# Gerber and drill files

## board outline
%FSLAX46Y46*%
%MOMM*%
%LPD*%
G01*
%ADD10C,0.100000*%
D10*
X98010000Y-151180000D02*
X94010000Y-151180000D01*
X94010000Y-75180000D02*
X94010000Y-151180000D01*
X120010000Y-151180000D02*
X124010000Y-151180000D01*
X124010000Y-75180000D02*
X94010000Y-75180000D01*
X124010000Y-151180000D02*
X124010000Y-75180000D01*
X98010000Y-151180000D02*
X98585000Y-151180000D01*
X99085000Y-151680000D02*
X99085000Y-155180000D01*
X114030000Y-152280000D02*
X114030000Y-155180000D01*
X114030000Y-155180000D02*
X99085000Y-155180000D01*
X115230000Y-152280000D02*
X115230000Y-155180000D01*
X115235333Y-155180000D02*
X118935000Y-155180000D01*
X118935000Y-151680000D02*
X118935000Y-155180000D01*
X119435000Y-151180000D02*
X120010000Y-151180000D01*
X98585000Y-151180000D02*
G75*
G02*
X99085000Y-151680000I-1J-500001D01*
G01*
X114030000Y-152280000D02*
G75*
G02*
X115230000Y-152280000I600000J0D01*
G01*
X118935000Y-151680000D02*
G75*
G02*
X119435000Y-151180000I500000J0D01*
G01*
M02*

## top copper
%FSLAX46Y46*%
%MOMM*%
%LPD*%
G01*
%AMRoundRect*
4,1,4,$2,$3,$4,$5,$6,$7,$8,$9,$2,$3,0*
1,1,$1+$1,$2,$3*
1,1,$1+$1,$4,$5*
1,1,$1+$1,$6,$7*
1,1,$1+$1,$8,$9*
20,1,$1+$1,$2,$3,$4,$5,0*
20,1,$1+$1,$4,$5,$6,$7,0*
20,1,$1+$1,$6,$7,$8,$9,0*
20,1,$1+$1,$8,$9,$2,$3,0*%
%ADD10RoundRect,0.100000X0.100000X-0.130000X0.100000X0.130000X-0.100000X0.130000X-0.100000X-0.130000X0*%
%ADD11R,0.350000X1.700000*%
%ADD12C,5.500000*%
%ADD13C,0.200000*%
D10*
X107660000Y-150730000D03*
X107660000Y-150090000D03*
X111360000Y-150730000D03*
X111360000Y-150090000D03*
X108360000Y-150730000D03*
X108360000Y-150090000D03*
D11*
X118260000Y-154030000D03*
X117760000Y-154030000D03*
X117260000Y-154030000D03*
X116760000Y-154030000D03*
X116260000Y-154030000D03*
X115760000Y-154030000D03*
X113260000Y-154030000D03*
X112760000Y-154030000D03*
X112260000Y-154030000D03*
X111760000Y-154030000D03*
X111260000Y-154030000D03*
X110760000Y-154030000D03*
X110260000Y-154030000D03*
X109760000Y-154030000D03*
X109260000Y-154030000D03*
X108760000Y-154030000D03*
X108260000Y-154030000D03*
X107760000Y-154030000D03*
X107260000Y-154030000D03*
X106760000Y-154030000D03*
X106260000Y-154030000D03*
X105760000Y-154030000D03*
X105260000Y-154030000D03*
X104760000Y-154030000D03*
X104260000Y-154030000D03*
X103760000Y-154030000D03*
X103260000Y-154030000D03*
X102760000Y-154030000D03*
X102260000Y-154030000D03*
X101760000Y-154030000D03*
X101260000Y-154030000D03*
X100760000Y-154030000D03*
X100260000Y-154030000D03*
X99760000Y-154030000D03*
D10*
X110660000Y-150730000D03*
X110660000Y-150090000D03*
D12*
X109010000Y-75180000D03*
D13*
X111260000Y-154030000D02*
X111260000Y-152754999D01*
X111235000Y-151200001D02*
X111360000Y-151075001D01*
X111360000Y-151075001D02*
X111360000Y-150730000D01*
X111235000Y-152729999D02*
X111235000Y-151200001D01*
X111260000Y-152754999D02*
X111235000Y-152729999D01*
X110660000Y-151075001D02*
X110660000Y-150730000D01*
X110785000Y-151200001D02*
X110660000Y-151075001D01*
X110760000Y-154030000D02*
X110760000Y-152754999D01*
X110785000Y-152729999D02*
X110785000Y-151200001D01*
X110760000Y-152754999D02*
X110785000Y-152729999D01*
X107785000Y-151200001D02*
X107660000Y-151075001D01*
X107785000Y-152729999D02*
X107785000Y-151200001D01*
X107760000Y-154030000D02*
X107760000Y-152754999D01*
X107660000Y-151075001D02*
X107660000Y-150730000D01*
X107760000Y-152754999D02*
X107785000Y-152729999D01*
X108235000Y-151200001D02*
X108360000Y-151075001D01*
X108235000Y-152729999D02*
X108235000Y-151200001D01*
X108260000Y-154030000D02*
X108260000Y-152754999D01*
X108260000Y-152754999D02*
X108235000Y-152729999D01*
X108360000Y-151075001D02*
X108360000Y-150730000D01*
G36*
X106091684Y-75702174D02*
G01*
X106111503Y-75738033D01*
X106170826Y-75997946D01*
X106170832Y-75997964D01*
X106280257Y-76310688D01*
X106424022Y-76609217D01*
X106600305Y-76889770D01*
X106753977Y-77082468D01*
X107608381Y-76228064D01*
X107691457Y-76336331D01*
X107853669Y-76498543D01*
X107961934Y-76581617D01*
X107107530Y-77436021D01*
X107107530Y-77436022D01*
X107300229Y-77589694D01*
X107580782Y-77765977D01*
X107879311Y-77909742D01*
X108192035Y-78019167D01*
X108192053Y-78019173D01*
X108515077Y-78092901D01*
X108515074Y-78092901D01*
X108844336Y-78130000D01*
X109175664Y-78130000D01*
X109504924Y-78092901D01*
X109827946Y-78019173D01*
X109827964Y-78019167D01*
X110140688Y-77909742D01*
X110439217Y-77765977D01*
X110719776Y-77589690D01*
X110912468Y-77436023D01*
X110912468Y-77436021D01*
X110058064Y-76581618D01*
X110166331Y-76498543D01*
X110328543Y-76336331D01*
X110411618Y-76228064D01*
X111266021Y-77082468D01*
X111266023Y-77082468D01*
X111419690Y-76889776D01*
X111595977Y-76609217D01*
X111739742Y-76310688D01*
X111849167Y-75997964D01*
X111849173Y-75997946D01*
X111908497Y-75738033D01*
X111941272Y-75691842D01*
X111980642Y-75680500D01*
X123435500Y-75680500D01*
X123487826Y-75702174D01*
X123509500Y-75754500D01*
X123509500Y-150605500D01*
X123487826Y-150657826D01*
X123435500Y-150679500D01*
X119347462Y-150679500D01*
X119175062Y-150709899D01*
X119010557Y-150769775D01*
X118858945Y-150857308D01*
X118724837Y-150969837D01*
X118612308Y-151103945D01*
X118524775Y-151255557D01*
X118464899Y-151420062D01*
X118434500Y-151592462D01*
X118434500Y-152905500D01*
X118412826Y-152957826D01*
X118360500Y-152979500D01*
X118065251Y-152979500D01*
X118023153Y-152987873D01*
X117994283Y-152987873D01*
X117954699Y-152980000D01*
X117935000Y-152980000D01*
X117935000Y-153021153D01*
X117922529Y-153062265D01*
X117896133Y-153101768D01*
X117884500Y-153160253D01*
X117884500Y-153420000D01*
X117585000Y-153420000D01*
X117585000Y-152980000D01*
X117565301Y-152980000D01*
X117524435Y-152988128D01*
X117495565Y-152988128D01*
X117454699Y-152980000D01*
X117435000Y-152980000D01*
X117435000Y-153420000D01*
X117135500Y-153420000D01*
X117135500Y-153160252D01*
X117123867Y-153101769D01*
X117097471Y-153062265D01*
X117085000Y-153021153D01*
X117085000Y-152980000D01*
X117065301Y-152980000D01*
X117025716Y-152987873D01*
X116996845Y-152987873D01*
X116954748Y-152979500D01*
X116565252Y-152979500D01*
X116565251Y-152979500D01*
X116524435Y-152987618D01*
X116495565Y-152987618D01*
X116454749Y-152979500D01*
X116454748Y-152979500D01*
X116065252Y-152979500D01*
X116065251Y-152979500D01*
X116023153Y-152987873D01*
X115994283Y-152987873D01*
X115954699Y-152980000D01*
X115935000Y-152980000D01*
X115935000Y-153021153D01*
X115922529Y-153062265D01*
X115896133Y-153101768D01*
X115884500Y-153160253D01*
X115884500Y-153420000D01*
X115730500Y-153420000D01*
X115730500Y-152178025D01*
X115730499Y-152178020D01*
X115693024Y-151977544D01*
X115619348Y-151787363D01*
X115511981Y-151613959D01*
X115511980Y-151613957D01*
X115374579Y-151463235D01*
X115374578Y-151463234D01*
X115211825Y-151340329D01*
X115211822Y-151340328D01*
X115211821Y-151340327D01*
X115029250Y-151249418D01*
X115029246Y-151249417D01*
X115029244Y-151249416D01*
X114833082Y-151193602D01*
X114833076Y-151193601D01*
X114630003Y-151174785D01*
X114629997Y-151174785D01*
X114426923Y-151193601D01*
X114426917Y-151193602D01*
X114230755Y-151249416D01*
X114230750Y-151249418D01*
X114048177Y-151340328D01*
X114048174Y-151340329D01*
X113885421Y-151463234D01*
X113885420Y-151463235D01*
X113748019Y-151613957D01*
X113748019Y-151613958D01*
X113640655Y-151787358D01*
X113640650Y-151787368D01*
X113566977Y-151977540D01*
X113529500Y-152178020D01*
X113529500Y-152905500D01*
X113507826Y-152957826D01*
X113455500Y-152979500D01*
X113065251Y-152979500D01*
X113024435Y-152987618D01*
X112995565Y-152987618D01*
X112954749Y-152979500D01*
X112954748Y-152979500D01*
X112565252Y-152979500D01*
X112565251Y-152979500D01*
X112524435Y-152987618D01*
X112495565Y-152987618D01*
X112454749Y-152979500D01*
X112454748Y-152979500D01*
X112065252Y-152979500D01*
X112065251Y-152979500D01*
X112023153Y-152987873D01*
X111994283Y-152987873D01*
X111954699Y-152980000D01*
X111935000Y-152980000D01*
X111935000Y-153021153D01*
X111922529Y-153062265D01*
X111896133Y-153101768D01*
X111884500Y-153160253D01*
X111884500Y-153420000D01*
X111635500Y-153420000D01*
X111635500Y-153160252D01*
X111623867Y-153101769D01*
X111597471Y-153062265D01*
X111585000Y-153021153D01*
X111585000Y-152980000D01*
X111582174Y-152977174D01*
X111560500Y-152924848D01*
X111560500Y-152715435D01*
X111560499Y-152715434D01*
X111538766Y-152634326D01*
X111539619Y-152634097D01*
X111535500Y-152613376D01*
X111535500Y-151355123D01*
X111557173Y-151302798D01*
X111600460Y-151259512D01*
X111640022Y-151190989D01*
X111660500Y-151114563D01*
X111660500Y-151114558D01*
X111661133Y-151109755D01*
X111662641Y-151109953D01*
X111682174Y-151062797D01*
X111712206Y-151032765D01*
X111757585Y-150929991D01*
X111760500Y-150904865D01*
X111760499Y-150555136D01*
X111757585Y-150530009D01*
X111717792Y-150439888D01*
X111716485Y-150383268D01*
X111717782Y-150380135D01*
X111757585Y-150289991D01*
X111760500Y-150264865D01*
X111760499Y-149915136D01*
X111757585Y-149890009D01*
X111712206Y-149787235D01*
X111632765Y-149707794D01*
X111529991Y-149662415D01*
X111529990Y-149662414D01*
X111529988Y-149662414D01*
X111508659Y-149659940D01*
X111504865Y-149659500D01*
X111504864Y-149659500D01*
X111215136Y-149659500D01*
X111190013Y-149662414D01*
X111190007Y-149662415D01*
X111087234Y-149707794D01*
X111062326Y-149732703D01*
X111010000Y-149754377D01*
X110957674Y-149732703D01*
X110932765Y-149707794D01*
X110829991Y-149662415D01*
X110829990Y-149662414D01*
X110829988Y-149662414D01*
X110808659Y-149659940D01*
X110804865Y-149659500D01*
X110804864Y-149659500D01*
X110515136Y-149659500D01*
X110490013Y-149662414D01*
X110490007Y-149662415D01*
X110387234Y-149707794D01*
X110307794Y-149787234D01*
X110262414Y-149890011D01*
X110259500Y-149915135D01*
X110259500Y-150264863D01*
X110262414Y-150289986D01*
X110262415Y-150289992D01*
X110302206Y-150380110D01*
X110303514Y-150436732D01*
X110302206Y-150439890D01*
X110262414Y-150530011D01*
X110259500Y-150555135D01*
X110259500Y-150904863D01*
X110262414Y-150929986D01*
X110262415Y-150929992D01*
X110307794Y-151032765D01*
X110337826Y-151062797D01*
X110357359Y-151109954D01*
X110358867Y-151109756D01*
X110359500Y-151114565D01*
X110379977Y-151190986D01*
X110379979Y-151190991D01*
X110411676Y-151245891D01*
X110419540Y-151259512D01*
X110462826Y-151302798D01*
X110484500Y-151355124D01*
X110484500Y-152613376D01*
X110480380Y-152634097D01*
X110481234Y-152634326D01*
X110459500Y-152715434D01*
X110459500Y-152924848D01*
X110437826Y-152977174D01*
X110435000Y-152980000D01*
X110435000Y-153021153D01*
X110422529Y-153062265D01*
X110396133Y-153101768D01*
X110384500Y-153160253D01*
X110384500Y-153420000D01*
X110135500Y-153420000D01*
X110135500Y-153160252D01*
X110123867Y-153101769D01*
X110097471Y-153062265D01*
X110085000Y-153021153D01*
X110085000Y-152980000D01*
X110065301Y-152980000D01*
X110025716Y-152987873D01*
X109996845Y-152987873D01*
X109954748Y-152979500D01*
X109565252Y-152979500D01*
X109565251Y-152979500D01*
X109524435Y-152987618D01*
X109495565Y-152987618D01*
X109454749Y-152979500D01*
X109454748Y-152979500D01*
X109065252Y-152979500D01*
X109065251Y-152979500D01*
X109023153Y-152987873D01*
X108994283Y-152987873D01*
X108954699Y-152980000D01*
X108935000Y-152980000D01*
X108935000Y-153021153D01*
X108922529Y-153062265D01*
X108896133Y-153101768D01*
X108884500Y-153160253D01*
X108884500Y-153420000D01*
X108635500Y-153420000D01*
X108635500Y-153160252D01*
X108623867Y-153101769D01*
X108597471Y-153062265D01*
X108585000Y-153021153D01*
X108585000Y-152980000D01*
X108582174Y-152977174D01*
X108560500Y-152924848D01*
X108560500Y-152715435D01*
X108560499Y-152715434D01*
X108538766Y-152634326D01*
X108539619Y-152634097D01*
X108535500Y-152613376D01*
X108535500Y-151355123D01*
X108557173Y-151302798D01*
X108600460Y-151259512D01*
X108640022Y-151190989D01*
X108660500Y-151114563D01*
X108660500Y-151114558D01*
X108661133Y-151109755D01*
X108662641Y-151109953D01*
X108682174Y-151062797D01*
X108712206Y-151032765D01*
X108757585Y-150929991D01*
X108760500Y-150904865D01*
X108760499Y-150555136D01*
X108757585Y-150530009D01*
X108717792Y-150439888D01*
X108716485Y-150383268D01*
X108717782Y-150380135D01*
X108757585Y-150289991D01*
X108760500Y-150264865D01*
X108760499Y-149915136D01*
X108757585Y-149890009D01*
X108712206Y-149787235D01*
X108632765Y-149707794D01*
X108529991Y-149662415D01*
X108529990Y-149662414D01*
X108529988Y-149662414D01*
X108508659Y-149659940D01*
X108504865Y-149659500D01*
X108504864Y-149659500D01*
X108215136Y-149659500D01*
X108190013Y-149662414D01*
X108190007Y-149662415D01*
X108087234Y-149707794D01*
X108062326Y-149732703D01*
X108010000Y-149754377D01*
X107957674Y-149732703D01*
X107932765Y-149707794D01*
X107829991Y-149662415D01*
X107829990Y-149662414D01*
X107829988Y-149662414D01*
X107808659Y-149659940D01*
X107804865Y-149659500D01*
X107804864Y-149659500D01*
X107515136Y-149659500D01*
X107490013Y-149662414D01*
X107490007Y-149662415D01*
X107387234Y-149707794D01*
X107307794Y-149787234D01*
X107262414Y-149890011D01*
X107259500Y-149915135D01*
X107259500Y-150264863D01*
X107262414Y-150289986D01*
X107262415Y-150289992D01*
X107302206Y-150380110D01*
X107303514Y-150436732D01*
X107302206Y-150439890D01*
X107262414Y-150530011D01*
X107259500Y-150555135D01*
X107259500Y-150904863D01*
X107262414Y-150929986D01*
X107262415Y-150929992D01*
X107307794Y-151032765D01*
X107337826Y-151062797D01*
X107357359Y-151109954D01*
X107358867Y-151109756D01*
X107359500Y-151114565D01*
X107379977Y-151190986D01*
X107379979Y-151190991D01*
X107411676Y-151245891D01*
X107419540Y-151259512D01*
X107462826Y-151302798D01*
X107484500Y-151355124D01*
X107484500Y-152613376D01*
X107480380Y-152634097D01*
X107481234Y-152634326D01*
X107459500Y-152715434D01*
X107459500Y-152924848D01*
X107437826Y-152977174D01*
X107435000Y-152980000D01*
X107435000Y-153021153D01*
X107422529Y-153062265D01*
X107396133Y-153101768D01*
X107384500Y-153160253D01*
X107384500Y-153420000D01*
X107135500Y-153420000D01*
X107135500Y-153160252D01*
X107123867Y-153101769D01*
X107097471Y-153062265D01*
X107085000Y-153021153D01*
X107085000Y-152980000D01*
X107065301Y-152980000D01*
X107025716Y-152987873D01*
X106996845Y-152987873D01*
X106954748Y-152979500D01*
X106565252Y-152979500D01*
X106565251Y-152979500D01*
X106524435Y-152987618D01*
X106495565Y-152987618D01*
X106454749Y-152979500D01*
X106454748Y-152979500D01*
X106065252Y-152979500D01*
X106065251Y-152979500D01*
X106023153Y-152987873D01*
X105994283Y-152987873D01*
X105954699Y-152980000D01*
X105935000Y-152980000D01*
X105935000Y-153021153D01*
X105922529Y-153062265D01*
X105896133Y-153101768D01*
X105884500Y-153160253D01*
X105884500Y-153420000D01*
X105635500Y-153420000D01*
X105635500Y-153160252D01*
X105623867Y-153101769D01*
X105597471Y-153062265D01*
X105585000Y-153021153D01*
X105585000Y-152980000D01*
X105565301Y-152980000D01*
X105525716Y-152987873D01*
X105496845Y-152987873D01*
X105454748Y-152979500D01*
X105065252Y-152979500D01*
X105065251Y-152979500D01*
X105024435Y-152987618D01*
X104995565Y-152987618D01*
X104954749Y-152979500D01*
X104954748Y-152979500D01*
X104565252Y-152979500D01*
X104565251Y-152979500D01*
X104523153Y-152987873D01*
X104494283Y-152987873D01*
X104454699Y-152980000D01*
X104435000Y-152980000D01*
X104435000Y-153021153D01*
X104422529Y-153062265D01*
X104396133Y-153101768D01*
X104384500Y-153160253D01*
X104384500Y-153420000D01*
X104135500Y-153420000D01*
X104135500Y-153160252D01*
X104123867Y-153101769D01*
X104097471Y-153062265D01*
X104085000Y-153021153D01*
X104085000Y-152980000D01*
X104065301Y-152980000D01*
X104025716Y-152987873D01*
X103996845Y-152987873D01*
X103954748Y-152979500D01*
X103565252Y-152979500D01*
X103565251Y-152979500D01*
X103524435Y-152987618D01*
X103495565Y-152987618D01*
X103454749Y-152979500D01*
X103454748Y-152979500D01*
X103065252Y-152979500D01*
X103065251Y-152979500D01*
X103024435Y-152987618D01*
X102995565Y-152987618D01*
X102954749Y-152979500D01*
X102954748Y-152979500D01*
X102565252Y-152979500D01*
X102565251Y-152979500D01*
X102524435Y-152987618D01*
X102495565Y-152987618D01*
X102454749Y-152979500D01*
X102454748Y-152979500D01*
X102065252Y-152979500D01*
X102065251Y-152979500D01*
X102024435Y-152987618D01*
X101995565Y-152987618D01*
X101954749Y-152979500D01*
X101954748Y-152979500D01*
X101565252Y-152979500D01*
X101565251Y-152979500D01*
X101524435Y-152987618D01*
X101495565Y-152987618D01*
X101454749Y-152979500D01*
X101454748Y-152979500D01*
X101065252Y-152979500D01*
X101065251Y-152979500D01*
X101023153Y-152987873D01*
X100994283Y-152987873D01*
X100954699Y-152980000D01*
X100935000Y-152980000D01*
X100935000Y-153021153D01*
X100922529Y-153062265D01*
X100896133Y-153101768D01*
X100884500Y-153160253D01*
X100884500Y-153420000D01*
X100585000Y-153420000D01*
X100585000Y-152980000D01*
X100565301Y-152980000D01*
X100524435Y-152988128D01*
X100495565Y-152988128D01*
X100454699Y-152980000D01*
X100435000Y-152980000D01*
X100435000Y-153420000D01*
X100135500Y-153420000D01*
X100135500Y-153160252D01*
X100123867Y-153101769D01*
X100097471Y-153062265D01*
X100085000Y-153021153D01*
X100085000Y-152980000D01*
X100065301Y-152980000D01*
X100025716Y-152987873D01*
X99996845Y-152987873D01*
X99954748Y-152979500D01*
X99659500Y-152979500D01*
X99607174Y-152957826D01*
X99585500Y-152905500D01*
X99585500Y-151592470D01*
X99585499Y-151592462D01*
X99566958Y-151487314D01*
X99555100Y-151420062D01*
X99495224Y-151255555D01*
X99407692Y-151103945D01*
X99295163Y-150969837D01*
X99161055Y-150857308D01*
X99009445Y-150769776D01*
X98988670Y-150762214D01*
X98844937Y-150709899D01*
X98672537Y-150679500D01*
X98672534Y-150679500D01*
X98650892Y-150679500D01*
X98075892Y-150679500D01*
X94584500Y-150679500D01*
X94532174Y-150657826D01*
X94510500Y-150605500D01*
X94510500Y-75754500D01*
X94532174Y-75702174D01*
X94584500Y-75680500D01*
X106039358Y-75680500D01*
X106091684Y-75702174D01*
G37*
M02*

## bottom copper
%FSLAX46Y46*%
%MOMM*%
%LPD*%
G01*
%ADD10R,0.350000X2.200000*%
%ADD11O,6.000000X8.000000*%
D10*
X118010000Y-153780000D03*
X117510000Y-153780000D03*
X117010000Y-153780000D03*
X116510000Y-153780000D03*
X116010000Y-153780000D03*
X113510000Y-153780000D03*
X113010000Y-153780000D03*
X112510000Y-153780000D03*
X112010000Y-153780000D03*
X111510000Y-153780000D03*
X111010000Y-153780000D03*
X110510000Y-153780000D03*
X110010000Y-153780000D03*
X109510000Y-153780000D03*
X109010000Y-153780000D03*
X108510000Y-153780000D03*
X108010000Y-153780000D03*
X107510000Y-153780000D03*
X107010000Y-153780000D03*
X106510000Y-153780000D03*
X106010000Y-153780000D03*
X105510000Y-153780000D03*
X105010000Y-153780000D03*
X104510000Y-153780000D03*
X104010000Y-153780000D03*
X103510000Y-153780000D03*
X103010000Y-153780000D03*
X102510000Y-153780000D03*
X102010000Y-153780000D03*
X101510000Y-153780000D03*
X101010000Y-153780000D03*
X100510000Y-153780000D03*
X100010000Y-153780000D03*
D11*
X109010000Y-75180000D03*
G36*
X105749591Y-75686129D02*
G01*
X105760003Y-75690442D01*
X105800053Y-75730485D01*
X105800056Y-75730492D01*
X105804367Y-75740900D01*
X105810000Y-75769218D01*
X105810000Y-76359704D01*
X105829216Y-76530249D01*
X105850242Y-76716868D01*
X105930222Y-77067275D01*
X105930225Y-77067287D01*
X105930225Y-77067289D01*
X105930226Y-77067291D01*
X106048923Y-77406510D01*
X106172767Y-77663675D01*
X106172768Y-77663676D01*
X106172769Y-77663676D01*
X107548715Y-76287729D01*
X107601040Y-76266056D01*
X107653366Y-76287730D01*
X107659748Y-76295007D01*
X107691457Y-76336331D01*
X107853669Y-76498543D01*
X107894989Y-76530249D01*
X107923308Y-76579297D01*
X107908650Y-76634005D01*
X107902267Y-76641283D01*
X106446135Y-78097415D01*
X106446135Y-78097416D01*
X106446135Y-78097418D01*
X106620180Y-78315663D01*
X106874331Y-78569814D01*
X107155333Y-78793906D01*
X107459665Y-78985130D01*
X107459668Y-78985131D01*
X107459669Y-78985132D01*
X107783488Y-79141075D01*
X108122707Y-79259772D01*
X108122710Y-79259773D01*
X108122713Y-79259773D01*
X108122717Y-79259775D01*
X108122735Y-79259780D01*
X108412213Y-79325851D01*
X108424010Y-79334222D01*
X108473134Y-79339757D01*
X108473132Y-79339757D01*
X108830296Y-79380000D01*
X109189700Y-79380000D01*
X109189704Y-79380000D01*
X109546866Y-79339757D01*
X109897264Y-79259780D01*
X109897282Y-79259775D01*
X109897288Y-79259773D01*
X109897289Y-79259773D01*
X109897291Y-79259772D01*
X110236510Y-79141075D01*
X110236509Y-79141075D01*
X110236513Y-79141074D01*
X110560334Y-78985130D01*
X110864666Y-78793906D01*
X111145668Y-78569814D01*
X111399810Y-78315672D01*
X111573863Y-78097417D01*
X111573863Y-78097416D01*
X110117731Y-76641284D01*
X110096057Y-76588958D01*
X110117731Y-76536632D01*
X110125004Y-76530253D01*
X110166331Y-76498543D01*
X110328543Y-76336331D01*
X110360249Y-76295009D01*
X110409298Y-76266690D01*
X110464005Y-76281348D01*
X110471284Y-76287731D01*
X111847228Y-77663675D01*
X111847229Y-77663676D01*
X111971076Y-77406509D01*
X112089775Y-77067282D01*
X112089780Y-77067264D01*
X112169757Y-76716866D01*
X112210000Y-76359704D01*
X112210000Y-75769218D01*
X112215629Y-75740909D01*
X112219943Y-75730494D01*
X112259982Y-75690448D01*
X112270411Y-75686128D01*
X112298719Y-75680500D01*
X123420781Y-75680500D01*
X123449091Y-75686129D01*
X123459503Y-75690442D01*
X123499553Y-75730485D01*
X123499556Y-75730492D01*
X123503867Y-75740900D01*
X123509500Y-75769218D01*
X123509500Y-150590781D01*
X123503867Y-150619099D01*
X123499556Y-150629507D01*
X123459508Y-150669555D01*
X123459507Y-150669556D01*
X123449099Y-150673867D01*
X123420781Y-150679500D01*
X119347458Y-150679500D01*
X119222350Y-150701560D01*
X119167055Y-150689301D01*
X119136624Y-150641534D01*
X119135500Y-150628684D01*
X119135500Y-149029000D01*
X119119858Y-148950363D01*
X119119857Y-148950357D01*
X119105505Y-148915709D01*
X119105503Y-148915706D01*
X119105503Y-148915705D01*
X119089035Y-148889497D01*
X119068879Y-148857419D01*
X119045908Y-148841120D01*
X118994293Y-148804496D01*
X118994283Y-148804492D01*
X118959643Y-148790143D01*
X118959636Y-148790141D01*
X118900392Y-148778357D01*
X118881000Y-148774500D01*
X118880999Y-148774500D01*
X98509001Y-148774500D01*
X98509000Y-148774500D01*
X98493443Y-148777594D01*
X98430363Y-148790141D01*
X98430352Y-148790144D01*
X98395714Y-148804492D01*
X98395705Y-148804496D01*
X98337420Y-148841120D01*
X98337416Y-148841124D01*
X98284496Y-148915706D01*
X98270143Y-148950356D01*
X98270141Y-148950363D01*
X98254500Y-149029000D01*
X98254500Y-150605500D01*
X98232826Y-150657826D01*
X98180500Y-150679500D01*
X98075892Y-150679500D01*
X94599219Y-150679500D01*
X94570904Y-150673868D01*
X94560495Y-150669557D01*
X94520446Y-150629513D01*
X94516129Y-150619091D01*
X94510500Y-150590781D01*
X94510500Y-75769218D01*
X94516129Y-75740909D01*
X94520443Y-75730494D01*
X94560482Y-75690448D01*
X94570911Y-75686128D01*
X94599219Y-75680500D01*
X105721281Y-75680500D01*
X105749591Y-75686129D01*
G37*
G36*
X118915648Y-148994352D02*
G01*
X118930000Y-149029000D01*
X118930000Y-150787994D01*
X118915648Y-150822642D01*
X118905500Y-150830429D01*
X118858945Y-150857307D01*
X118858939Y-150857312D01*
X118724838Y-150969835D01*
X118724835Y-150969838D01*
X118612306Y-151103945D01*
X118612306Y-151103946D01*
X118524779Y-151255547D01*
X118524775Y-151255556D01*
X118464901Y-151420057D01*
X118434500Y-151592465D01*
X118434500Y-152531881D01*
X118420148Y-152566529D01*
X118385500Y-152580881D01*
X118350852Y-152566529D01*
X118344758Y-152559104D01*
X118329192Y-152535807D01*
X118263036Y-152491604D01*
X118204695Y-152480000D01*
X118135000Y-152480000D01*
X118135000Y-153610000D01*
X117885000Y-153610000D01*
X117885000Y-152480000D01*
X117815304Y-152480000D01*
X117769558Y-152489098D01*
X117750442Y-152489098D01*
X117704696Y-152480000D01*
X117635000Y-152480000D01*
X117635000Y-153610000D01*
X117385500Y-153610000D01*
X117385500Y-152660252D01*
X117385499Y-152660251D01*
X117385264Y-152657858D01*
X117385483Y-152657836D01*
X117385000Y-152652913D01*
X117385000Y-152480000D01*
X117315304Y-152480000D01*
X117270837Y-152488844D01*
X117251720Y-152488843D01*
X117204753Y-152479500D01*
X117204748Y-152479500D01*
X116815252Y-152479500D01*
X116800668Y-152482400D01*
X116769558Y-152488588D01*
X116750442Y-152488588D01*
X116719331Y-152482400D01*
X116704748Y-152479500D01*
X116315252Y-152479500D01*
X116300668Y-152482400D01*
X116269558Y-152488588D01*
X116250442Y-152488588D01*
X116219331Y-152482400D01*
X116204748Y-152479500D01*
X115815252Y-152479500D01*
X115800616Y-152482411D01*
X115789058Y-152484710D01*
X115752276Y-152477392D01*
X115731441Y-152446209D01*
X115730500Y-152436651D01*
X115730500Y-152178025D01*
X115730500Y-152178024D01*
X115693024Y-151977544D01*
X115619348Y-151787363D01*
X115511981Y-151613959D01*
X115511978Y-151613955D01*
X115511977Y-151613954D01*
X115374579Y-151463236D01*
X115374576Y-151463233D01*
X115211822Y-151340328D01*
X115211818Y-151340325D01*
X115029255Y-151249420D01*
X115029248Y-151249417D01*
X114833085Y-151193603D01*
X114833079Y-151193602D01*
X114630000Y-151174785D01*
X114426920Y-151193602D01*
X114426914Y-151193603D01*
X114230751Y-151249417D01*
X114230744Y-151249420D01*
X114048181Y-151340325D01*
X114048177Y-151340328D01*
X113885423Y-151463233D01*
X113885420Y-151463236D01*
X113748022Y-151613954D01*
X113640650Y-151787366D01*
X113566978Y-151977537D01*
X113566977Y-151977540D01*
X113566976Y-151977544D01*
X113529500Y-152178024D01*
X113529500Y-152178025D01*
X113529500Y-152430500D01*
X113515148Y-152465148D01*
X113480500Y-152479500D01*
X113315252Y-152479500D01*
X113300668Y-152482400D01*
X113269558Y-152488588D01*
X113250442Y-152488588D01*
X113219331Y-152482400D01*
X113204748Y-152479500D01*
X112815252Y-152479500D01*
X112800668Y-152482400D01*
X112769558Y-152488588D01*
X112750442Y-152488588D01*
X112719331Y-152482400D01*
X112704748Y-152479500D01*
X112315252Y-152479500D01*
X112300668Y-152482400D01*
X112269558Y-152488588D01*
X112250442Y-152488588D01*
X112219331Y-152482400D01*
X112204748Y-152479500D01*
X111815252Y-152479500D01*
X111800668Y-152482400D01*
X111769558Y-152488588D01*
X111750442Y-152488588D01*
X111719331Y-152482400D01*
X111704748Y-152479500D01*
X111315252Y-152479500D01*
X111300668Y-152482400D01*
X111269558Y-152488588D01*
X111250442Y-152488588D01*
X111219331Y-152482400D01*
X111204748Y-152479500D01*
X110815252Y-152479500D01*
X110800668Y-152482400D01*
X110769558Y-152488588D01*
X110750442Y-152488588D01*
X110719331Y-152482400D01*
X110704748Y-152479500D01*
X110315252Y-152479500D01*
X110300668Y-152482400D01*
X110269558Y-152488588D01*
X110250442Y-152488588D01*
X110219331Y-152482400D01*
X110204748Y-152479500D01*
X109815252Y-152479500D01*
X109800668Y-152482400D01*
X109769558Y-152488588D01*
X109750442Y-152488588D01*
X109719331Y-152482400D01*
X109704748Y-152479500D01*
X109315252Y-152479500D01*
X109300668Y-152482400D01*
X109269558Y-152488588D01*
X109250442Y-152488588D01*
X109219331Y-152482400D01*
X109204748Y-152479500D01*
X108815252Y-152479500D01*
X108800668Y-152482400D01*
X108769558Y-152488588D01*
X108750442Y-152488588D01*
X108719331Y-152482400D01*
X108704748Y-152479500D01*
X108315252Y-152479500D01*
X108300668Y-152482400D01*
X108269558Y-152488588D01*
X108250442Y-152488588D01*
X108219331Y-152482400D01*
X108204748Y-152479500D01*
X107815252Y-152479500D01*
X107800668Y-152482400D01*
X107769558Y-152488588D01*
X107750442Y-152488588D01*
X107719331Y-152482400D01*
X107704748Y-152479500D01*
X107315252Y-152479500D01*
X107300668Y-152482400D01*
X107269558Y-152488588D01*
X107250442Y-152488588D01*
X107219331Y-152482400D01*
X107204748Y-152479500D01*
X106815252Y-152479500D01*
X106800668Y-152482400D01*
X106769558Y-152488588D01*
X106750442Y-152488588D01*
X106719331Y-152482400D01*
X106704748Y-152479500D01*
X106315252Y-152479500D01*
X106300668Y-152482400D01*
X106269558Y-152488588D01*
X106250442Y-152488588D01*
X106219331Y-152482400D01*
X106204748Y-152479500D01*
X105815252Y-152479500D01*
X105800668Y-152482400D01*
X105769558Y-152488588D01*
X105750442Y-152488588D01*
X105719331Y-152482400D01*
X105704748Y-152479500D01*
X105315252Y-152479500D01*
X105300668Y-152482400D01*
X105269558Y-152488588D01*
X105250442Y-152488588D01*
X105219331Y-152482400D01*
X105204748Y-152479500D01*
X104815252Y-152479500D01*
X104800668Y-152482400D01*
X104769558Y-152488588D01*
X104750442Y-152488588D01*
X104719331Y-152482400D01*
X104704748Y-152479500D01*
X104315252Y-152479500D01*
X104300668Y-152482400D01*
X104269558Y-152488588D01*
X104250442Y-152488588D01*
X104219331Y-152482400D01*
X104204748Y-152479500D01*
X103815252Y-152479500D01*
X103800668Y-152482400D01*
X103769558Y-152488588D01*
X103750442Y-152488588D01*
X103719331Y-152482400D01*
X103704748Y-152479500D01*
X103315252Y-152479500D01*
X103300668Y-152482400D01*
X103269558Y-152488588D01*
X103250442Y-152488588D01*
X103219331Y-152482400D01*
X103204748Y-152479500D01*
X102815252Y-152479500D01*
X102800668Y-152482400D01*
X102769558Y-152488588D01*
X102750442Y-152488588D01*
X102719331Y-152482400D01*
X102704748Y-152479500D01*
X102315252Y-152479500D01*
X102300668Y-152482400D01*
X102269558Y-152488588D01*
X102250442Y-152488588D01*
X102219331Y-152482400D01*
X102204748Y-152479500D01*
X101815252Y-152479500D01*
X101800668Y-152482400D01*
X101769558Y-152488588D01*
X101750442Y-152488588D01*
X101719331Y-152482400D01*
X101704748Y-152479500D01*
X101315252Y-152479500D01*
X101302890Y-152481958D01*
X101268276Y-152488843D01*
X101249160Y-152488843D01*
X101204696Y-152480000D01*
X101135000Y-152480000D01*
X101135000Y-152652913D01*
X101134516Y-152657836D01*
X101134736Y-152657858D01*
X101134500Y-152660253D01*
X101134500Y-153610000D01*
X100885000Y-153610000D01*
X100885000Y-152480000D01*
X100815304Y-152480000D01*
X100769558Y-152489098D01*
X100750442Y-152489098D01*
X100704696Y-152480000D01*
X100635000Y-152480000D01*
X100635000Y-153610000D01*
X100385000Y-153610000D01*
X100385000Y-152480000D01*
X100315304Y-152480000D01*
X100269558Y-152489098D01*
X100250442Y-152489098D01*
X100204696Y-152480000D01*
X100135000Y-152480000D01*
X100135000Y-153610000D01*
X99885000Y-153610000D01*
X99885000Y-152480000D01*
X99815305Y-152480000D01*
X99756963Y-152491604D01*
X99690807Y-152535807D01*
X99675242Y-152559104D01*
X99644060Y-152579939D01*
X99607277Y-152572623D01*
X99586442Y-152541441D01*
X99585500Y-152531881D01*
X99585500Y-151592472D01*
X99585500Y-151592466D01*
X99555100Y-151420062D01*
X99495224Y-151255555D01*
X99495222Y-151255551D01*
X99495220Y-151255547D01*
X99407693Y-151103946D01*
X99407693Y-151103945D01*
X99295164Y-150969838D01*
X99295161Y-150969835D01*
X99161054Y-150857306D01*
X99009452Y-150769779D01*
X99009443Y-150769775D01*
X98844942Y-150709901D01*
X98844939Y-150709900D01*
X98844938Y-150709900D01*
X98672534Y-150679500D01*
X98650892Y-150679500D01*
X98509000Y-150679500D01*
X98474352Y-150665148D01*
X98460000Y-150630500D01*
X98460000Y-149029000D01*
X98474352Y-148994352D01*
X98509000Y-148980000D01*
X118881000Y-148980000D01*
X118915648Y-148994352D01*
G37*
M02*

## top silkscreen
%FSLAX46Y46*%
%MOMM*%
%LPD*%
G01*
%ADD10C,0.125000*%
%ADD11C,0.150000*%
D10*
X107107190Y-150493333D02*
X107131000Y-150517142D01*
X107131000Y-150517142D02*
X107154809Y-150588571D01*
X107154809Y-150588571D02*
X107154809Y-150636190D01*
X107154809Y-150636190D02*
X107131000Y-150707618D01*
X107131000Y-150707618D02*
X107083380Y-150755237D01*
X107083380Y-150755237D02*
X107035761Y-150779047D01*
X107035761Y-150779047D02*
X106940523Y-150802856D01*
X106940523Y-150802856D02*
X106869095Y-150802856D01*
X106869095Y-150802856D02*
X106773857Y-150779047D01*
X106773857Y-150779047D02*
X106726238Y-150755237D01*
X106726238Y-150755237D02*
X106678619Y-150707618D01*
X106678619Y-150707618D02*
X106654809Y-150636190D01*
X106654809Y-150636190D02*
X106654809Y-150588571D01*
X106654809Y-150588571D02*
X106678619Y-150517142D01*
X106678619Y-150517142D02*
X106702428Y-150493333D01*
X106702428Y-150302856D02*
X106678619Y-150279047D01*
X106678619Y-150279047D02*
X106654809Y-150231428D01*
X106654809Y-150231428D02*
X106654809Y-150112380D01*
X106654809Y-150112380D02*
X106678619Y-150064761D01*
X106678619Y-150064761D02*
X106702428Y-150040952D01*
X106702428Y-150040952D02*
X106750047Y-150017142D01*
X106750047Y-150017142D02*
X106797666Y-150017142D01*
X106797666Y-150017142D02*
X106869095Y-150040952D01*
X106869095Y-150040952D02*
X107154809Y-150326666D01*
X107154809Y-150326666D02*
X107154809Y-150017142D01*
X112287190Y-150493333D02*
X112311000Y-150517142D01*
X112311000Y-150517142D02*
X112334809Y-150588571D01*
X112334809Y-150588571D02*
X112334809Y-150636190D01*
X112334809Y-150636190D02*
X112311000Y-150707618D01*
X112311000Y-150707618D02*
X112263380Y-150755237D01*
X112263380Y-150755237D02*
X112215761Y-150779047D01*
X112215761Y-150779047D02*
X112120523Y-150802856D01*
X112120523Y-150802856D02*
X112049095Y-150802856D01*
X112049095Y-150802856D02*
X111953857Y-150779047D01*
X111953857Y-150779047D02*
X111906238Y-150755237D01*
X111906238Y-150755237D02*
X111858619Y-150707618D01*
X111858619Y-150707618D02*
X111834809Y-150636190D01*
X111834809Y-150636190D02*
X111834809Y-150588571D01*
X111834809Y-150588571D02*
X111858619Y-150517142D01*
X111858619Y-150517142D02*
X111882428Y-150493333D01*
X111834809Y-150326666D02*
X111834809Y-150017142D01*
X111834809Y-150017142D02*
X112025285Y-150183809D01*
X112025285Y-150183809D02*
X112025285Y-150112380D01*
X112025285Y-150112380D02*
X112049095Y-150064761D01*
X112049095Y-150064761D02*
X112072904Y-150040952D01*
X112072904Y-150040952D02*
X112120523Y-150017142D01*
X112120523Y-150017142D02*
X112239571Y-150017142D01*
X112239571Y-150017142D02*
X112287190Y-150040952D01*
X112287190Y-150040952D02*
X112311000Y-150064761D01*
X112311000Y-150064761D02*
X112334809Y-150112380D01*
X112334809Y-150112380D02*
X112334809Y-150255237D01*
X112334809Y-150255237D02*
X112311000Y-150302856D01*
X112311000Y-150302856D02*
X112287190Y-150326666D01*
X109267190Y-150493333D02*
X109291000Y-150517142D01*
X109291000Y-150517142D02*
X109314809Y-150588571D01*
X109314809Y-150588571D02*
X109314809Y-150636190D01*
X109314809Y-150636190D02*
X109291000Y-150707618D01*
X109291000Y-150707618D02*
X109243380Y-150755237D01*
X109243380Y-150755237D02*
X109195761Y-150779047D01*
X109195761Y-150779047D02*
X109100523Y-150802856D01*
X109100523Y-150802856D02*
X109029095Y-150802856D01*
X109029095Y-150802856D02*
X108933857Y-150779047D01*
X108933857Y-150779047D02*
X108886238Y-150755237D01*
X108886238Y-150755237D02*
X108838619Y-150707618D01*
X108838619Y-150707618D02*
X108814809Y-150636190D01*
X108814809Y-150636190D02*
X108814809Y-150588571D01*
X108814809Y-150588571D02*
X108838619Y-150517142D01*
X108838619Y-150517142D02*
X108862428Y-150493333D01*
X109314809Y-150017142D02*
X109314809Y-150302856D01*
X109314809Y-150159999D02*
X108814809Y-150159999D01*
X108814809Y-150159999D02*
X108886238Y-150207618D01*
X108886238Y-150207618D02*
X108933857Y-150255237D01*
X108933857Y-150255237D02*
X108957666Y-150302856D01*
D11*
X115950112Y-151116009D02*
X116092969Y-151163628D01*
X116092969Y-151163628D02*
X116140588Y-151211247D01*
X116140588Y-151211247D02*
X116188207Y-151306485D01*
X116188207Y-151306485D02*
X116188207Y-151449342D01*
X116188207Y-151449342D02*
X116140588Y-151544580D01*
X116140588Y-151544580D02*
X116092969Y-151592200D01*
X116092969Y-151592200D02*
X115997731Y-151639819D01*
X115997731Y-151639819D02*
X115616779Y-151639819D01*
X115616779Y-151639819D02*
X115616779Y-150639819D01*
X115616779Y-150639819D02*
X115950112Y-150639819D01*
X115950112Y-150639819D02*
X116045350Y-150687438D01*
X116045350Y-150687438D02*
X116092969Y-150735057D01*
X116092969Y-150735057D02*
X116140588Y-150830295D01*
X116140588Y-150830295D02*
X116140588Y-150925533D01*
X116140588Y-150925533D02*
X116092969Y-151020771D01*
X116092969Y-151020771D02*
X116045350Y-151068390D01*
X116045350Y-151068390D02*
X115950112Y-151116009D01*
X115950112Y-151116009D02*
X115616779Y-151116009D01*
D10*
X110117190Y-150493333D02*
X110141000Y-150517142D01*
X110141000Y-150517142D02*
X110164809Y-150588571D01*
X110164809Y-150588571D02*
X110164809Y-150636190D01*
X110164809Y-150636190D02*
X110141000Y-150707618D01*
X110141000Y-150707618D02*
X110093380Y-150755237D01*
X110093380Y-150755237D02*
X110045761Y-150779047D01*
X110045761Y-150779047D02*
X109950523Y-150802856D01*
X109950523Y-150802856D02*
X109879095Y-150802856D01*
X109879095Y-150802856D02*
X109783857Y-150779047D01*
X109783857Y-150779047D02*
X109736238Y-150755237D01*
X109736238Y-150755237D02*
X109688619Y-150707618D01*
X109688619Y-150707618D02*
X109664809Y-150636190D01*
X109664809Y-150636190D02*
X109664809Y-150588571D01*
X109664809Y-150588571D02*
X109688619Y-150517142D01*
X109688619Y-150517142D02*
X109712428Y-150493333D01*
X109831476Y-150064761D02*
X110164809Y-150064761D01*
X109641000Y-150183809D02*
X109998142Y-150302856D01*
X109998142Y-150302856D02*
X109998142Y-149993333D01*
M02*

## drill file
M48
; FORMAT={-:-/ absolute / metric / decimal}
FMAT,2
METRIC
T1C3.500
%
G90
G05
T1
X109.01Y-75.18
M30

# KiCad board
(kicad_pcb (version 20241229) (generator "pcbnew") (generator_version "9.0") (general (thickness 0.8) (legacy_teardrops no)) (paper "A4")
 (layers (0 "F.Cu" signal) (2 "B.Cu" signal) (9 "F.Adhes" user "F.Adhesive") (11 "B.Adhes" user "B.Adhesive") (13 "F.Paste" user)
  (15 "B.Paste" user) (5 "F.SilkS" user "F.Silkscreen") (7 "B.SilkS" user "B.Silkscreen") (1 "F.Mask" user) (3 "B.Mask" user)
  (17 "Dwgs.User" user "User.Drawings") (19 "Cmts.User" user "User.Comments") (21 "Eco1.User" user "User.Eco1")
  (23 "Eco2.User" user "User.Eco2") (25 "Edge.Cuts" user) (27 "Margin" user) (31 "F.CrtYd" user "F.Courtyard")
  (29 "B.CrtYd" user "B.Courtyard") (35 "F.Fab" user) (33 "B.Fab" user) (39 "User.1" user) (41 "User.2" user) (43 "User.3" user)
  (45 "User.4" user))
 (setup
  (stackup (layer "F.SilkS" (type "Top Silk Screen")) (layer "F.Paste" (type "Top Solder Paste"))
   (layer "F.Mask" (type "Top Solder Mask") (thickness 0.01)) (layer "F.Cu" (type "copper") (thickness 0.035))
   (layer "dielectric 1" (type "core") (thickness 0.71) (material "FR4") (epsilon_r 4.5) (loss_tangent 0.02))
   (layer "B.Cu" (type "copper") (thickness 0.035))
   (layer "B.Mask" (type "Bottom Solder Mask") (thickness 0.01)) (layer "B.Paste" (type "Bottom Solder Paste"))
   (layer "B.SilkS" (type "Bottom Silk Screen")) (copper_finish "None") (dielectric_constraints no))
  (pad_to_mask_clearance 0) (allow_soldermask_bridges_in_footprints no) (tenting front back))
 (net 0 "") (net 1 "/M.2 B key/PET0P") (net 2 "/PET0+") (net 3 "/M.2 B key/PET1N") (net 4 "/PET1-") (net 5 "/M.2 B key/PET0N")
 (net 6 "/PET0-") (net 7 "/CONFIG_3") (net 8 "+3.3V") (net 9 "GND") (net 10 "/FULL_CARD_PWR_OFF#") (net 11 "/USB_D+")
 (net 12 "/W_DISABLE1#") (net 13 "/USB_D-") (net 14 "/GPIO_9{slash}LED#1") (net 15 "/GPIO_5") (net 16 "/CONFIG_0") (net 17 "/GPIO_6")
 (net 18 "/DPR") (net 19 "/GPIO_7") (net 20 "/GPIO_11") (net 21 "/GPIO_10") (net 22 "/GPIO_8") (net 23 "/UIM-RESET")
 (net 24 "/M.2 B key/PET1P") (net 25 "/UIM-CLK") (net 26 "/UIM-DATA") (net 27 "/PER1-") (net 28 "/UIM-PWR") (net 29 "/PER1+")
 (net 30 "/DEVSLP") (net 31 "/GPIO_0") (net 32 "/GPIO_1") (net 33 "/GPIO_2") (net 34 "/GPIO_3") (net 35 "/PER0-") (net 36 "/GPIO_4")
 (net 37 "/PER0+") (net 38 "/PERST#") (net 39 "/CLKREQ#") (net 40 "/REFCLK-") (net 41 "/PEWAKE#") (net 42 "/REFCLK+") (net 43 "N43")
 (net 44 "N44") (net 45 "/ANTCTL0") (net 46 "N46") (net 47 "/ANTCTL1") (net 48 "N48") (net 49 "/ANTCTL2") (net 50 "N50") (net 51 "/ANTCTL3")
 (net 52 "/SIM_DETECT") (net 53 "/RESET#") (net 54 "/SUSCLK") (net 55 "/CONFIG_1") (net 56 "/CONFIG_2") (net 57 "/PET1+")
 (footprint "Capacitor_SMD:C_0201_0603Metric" (layer "F.Cu") (at 107.66 150.41 90)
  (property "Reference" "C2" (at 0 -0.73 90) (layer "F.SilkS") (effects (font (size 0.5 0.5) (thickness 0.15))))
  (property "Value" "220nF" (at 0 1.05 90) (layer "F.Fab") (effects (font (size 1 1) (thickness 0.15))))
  (pad "" smd roundrect (at -0.345 0 90) (size 0.318 0.36) (layers "F.Paste") (roundrect_rratio 0.25))
  (pad "" smd roundrect (at 0.345 0 90) (size 0.318 0.36) (layers "F.Paste") (roundrect_rratio 0.25))
  (pad "1" smd roundrect (at -0.32 0 90) (size 0.46 0.4) (layers "F.Cu" "F.Mask") (roundrect_rratio 0.25) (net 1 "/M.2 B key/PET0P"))
  (pad "2" smd roundrect (at 0.32 0 90) (size 0.46 0.4) (layers "F.Cu" "F.Mask") (roundrect_rratio 0.25) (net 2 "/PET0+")))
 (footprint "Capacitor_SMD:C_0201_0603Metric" (layer "F.Cu") (at 111.36 150.41 90)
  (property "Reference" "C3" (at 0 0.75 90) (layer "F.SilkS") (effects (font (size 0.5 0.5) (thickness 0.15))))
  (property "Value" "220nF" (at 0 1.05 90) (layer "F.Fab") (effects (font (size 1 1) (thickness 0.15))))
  (pad "" smd roundrect (at -0.345 0 90) (size 0.318 0.36) (layers "F.Paste") (roundrect_rratio 0.25))
  (pad "" smd roundrect (at 0.345 0 90) (size 0.318 0.36) (layers "F.Paste") (roundrect_rratio 0.25))
  (pad "1" smd roundrect (at -0.32 0 90) (size 0.46 0.4) (layers "F.Cu" "F.Mask") (roundrect_rratio 0.25) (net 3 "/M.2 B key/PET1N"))
  (pad "2" smd roundrect (at 0.32 0 90) (size 0.46 0.4) (layers "F.Cu" "F.Mask") (roundrect_rratio 0.25) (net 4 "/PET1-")))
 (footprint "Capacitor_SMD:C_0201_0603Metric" (layer "F.Cu") (at 108.36 150.41 90)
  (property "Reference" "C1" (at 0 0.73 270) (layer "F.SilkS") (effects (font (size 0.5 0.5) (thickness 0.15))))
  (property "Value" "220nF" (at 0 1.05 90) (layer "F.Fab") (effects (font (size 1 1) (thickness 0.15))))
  (pad "" smd roundrect (at -0.345 0 90) (size 0.318 0.36) (layers "F.Paste") (roundrect_rratio 0.25))
  (pad "" smd roundrect (at 0.345 0 90) (size 0.318 0.36) (layers "F.Paste") (roundrect_rratio 0.25))
  (pad "1" smd roundrect (at -0.32 0 90) (size 0.46 0.4) (layers "F.Cu" "F.Mask") (roundrect_rratio 0.25) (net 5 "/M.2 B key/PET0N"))
  (pad "2" smd roundrect (at 0.32 0 90) (size 0.46 0.4) (layers "F.Cu" "F.Mask") (roundrect_rratio 0.25) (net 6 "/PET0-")))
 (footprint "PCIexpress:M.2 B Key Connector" (layer "F.Cu") (at 109.01 154.07)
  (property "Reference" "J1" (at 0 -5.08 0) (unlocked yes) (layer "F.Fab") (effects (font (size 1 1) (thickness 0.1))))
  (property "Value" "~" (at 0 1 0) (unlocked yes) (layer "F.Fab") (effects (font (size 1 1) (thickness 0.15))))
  (fp_line (start -11 -2.89) (end -10.425 -2.89) (stroke (width 0.1) (type default)) (layer "Edge.Cuts"))
  (fp_line (start -9.925 -2.39) (end -9.925 1.11) (stroke (width 0.1) (type default)) (layer "Edge.Cuts"))
  (fp_line (start 5.02 -1.79) (end 5.02 1.11) (stroke (width 0.1) (type default)) (layer "Edge.Cuts"))
  (fp_line (start 5.02 1.11) (end -9.925 1.11) (stroke (width 0.1) (type default)) (layer "Edge.Cuts"))
  (fp_line (start 6.22 -1.79) (end 6.22 1.11) (stroke (width 0.1) (type default)) (layer "Edge.Cuts"))
  (fp_line (start 6.225333 1.11) (end 9.925 1.11) (stroke (width 0.1) (type default)) (layer "Edge.Cuts"))
  (fp_line (start 9.925 -2.39) (end 9.925 1.11) (stroke (width 0.1) (type default)) (layer "Edge.Cuts"))
  (fp_line (start 10.425 -2.89) (end 11 -2.89) (stroke (width 0.1) (type default)) (layer "Edge.Cuts"))
  (fp_arc (start -10.425 -2.89) (mid -10.071447 -2.743553) (end -9.925 -2.39) (stroke (width 0.1) (type default)) (layer "Edge.Cuts"))
  (fp_arc (start 5.02 -1.79) (mid 5.62 -2.39) (end 6.22 -1.79) (stroke (width 0.1) (type default)) (layer "Edge.Cuts"))
  (fp_arc (start 9.925 -2.39) (mid 10.071447 -2.743553) (end 10.425 -2.89) (stroke (width 0.1) (type default)) (layer "Edge.Cuts"))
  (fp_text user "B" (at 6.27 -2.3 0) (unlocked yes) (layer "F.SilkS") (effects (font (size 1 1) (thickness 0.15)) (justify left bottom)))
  (pad "1" smd rect (at 9.25 -0.04 180) (size 0.35 1.7) (layers "F.Cu") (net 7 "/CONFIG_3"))
  (pad "2" smd rect (at 9 -0.29 180) (size 0.35 2.2) (layers "B.Cu") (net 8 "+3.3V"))
  (pad "3" smd rect (at 8.75 -0.04 180) (size 0.35 1.7) (layers "F.Cu") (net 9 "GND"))
  (pad "4" smd rect (at 8.5 -0.29 180) (size 0.35 2.2) (layers "B.Cu") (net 8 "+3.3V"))
  (pad "5" smd rect (at 8.25 -0.04 180) (size 0.35 1.7) (layers "F.Cu") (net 9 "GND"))
  (pad "6" smd rect (at 8 -0.29 180) (size 0.35 2.2) (layers "B.Cu") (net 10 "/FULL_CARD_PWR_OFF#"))
  (pad "7" smd rect (at 7.75 -0.04 180) (size 0.35 1.7) (layers "F.Cu") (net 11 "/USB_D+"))
  (pad "8" smd rect (at 7.5 -0.29 180) (size 0.35 2.2) (layers "B.Cu") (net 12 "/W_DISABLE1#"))
  (pad "9" smd rect (at 7.25 -0.04 180) (size 0.35 1.7) (layers "F.Cu") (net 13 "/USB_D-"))
  (pad "10" smd rect (at 7 -0.29 180) (size 0.35 2.2) (layers "B.Cu") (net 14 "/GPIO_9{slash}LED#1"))
  (pad "11" smd rect (at 6.75 -0.04 180) (size 0.35 1.7) (layers "F.Cu") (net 9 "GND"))
  (pad "20" smd rect (at 4.5 -0.29 180) (size 0.35 2.2) (layers "B.Cu") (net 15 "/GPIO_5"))
  (pad "21" smd rect (at 4.25 -0.04 180) (size 0.35 1.7) (layers "F.Cu") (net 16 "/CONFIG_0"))
  (pad "22" smd rect (at 4 -0.29 180) (size 0.35 2.2) (layers "B.Cu") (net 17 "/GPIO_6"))
  (pad "23" smd rect (at 3.75 -0.04 180) (size 0.35 1.7) (layers "F.Cu") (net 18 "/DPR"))
  (pad "24" smd rect (at 3.5 -0.29 180) (size 0.35 2.2) (layers "B.Cu") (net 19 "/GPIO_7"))
  (pad "25" smd rect (at 3.25 -0.04 180) (size 0.35 1.7) (layers "F.Cu") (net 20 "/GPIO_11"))
  (pad "26" smd rect (at 3 -0.29 180) (size 0.35 2.2) (layers "B.Cu") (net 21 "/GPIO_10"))
  (pad "27" smd rect (at 2.75 -0.04 180) (size 0.35 1.7) (layers "F.Cu") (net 9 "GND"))
  (pad "28" smd rect (at 2.5 -0.29 180) (size 0.35 2.2) (layers "B.Cu") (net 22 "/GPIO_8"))
  (pad "29" smd rect (at 2.25 -0.04 180) (size 0.35 1.7) (layers "F.Cu") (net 3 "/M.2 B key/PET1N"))
  (pad "30" smd rect (at 2 -0.29 180) (size 0.35 2.2) (layers "B.Cu") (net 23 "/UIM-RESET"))
  (pad "31" smd rect (at 1.75 -0.04 180) (size 0.35 1.7) (layers "F.Cu") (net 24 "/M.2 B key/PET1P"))
  (pad "32" smd rect (at 1.5 -0.29 180) (size 0.35 2.2) (layers "B.Cu") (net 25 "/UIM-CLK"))
  (pad "33" smd rect (at 1.25 -0.04 180) (size 0.35 1.7) (layers "F.Cu") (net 9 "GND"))
  (pad "34" smd rect (at 1 -0.29 180) (size 0.35 2.2) (layers "B.Cu") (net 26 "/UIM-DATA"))
  (pad "35" smd rect (at 0.75 -0.04 180) (size 0.35 1.7) (layers "F.Cu") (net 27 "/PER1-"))
  (pad "36" smd rect (at 0.5 -0.29 180) (size 0.35 2.2) (layers "B.Cu") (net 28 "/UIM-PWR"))
  (pad "37" smd rect (at 0.25 -0.04 180) (size 0.35 1.7) (layers "F.Cu") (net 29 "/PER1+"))
  (pad "38" smd rect (at 0 -0.29 180) (size 0.35 2.2) (layers "B.Cu") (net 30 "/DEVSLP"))
  (pad "39" smd rect (at -0.25 -0.04 180) (size 0.35 1.7) (layers "F.Cu") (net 9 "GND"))
  (pad "40" smd rect (at -0.5 -0.29 180) (size 0.35 2.2) (layers "B.Cu") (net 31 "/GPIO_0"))
  (pad "41" smd rect (at -0.75 -0.04 180) (size 0.35 1.7) (layers "F.Cu") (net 5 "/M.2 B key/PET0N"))
  (pad "42" smd rect (at -1 -0.29 180) (size 0.35 2.2) (layers "B.Cu") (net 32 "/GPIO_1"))
  (pad "43" smd rect (at -1.25 -0.04 180) (size 0.35 1.7) (layers "F.Cu") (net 1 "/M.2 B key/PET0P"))
  (pad "44" smd rect (at -1.5 -0.29 180) (size 0.35 2.2) (layers "B.Cu") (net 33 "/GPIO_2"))
  (pad "45" smd rect (at -1.75 -0.04 180) (size 0.35 1.7) (layers "F.Cu") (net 9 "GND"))
  (pad "46" smd rect (at -2 -0.29 180) (size 0.35 2.2) (layers "B.Cu") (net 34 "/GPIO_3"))
  (pad "47" smd rect (at -2.25 -0.04 180) (size 0.35 1.7) (layers "F.Cu") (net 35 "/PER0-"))
  (pad "48" smd rect (at -2.5 -0.29 180) (size 0.35 2.2) (layers "B.Cu") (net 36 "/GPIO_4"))
  (pad "49" smd rect (at -2.75 -0.04 180) (size 0.35 1.7) (layers "F.Cu") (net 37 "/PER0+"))
  (pad "50" smd rect (at -3 -0.29 180) (size 0.35 2.2) (layers "B.Cu") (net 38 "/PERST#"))
  (pad "51" smd rect (at -3.25 -0.04 180) (size 0.35 1.7) (layers "F.Cu") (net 9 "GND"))
  (pad "52" smd rect (at -3.5 -0.29 180) (size 0.35 2.2) (layers "B.Cu") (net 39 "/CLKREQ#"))
  (pad "53" smd rect (at -3.75 -0.04 180) (size 0.35 1.7) (layers "F.Cu") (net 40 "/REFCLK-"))
  (pad "54" smd rect (at -4 -0.29 180) (size 0.35 2.2) (layers "B.Cu") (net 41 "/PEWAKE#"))
  (pad "55" smd rect (at -4.25 -0.04 180) (size 0.35 1.7) (layers "F.Cu") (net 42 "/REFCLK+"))
  (pad "56" smd rect (at -4.5 -0.29 180) (size 0.35 2.2) (layers "B.Cu") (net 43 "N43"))
  (pad "57" smd rect (at -4.75 -0.04 180) (size 0.35 1.7) (layers "F.Cu") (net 9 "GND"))
  (pad "58" smd rect (at -5 -0.29 180) (size 0.35 2.2) (layers "B.Cu") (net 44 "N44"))
  (pad "59" smd rect (at -5.25 -0.04 180) (size 0.35 1.7) (layers "F.Cu") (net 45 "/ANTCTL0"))
  (pad "60" smd rect (at -5.5 -0.29 180) (size 0.35 2.2) (layers "B.Cu") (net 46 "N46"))
  (pad "61" smd rect (at -5.75 -0.04 180) (size 0.35 1.7) (layers "F.Cu") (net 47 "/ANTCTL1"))
  (pad "62" smd rect (at -6 -0.29 180) (size 0.35 2.2) (layers "B.Cu") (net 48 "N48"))
  (pad "63" smd rect (at -6.25 -0.04 180) (size 0.35 1.7) (layers "F.Cu") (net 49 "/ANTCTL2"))
  (pad "64" smd rect (at -6.5 -0.29 180) (size 0.35 2.2) (layers "B.Cu") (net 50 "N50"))
  (pad "65" smd rect (at -6.75 -0.04 180) (size 0.35 1.7) (layers "F.Cu") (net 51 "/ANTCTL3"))
  (pad "66" smd rect (at -7 -0.29 180) (size 0.35 2.2) (layers "B.Cu") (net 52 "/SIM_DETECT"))
  (pad "67" smd rect (at -7.25 -0.04 180) (size 0.35 1.7) (layers "F.Cu") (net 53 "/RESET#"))
  (pad "68" smd rect (at -7.5 -0.29 180) (size 0.35 2.2) (layers "B.Cu") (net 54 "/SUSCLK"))
  (pad "69" smd rect (at -7.75 -0.04 180) (size 0.35 1.7) (layers "F.Cu") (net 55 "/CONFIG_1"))
  (pad "70" smd rect (at -8 -0.29 180) (size 0.35 2.2) (layers "B.Cu") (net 8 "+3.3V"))
  (pad "71" smd rect (at -8.25 -0.04 180) (size 0.35 1.7) (layers "F.Cu") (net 9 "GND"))
  (pad "72" smd rect (at -8.5 -0.29 180) (size 0.35 2.2) (layers "B.Cu") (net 8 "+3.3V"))
  (pad "73" smd rect (at -8.75 -0.04 180) (size 0.35 1.7) (layers "F.Cu") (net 9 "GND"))
  (pad "74" smd rect (at -9 -0.29 180) (size 0.35 2.2) (layers "B.Cu") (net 8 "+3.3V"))
  (pad "75" smd rect (at -9.25 -0.04 180) (size 0.35 1.7) (layers "F.Cu") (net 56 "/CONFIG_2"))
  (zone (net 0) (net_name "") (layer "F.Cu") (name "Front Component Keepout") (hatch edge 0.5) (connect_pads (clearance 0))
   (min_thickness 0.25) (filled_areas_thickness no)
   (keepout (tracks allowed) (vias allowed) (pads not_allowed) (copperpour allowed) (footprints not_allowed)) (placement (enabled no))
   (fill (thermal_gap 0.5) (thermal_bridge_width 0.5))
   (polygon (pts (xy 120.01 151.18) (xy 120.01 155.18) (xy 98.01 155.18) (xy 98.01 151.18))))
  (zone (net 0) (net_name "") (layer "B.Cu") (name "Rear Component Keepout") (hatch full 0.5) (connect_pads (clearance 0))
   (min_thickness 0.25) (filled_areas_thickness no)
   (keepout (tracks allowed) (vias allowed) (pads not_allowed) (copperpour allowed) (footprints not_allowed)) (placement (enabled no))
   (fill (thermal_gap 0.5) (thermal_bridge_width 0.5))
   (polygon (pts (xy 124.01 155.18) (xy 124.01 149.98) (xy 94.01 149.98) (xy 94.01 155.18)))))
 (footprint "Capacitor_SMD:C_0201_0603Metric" (layer "F.Cu") (at 110.66 150.41 90)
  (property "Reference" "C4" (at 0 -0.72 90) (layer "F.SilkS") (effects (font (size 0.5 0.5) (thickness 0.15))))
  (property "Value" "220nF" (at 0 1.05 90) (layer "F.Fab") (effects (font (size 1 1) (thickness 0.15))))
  (pad "" smd roundrect (at -0.345 0 90) (size 0.318 0.36) (layers "F.Paste") (roundrect_rratio 0.25))
  (pad "" smd roundrect (at 0.345 0 90) (size 0.318 0.36) (layers "F.Paste") (roundrect_rratio 0.25))
  (pad "1" smd roundrect (at -0.32 0 90) (size 0.46 0.4) (layers "F.Cu" "F.Mask") (roundrect_rratio 0.25) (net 24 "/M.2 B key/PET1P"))
  (pad "2" smd roundrect (at 0.32 0 90) (size 0.46 0.4) (layers "F.Cu" "F.Mask") (roundrect_rratio 0.25) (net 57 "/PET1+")))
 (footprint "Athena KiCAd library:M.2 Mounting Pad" (layer "F.Cu") (at 109.01 75.18)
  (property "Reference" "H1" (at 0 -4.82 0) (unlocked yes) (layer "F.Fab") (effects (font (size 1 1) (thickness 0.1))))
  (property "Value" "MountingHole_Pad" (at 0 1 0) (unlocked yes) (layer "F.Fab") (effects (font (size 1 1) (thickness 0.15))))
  (pad "1" thru_hole circle (at 0 0) (size 5.5 5.5) (drill 3.5) (layers "*.Cu" "*.Mask") (remove_unused_layers no) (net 9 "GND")
   (padstack (mode front_inner_back)
    (layer "Inner" (shape circle) (size 5.5 5.5) (zone_connect -1))
    (layer "B.Cu" (shape oval) (size 6 8) (thermal_bridge_angle 45) (zone_connect -1)))))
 (gr_line (start 98.01 151.18) (end 94.01 151.18) (stroke (width 0.1) (type default)) (layer "Edge.Cuts"))
 (gr_line (start 94.01 75.18) (end 94.01 151.18) (stroke (width 0.1) (type default)) (layer "Edge.Cuts"))
 (gr_line (start 120.01 151.18) (end 124.01 151.18) (stroke (width 0.1) (type default)) (layer "Edge.Cuts"))
 (gr_line (start 124.01 75.18) (end 94.01 75.18) (stroke (width 0.1) (type default)) (layer "Edge.Cuts"))
 (gr_line (start 124.01 151.18) (end 124.01 75.18) (stroke (width 0.1) (type default)) (layer "Edge.Cuts"))
 (segment (start 111.26 154.03) (end 111.26 152.754999) (width 0.2) (layer "F.Cu") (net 3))
 (segment (start 111.235 151.200001) (end 111.36 151.075001) (width 0.2) (layer "F.Cu") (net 3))
 (segment (start 111.36 151.075001) (end 111.36 150.73) (width 0.2) (layer "F.Cu") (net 3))
 (segment (start 111.235 152.729999) (end 111.235 151.200001) (width 0.2) (layer "F.Cu") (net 3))
 (segment (start 111.26 152.754999) (end 111.235 152.729999) (width 0.2) (layer "F.Cu") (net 3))
 (segment (start 110.66 151.075001) (end 110.66 150.73) (width 0.2) (layer "F.Cu") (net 24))
 (segment (start 110.785 151.200001) (end 110.66 151.075001) (width 0.2) (layer "F.Cu") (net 24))
 (segment (start 110.76 154.03) (end 110.76 152.754999) (width 0.2) (layer "F.Cu") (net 24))
 (segment (start 110.785 152.729999) (end 110.785 151.200001) (width 0.2) (layer "F.Cu") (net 24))
 (segment (start 110.76 152.754999) (end 110.785 152.729999) (width 0.2) (layer "F.Cu") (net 24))
 (segment (start 107.785 151.200001) (end 107.66 151.075001) (width 0.2) (layer "F.Cu") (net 1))
 (segment (start 107.785 152.729999) (end 107.785 151.200001) (width 0.2) (layer "F.Cu") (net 1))
 (segment (start 107.76 154.03) (end 107.76 152.754999) (width 0.2) (layer "F.Cu") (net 1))
 (segment (start 107.66 151.075001) (end 107.66 150.73) (width 0.2) (layer "F.Cu") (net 1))
 (segment (start 107.76 152.754999) (end 107.785 152.729999) (width 0.2) (layer "F.Cu") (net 1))
 (segment (start 108.235 151.200001) (end 108.36 151.075001) (width 0.2) (layer "F.Cu") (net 5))
 (segment (start 108.235 152.729999) (end 108.235 151.200001) (width 0.2) (layer "F.Cu") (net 5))
 (segment (start 108.26 154.03) (end 108.26 152.754999) (width 0.2) (layer "F.Cu") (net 5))
 (segment (start 108.26 152.754999) (end 108.235 152.729999) (width 0.2) (layer "F.Cu") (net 5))
 (segment (start 108.36 151.075001) (end 108.36 150.73) (width 0.2) (layer "F.Cu") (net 5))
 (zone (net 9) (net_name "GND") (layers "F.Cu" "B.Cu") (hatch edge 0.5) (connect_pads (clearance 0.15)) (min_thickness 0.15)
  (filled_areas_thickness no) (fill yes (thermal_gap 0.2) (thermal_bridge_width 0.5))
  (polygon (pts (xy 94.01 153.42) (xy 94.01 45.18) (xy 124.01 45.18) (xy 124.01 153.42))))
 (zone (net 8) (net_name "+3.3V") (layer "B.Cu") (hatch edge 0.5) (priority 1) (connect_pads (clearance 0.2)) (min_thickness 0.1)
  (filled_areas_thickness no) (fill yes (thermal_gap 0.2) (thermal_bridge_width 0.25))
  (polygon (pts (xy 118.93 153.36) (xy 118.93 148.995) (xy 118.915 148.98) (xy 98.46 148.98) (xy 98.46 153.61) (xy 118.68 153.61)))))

